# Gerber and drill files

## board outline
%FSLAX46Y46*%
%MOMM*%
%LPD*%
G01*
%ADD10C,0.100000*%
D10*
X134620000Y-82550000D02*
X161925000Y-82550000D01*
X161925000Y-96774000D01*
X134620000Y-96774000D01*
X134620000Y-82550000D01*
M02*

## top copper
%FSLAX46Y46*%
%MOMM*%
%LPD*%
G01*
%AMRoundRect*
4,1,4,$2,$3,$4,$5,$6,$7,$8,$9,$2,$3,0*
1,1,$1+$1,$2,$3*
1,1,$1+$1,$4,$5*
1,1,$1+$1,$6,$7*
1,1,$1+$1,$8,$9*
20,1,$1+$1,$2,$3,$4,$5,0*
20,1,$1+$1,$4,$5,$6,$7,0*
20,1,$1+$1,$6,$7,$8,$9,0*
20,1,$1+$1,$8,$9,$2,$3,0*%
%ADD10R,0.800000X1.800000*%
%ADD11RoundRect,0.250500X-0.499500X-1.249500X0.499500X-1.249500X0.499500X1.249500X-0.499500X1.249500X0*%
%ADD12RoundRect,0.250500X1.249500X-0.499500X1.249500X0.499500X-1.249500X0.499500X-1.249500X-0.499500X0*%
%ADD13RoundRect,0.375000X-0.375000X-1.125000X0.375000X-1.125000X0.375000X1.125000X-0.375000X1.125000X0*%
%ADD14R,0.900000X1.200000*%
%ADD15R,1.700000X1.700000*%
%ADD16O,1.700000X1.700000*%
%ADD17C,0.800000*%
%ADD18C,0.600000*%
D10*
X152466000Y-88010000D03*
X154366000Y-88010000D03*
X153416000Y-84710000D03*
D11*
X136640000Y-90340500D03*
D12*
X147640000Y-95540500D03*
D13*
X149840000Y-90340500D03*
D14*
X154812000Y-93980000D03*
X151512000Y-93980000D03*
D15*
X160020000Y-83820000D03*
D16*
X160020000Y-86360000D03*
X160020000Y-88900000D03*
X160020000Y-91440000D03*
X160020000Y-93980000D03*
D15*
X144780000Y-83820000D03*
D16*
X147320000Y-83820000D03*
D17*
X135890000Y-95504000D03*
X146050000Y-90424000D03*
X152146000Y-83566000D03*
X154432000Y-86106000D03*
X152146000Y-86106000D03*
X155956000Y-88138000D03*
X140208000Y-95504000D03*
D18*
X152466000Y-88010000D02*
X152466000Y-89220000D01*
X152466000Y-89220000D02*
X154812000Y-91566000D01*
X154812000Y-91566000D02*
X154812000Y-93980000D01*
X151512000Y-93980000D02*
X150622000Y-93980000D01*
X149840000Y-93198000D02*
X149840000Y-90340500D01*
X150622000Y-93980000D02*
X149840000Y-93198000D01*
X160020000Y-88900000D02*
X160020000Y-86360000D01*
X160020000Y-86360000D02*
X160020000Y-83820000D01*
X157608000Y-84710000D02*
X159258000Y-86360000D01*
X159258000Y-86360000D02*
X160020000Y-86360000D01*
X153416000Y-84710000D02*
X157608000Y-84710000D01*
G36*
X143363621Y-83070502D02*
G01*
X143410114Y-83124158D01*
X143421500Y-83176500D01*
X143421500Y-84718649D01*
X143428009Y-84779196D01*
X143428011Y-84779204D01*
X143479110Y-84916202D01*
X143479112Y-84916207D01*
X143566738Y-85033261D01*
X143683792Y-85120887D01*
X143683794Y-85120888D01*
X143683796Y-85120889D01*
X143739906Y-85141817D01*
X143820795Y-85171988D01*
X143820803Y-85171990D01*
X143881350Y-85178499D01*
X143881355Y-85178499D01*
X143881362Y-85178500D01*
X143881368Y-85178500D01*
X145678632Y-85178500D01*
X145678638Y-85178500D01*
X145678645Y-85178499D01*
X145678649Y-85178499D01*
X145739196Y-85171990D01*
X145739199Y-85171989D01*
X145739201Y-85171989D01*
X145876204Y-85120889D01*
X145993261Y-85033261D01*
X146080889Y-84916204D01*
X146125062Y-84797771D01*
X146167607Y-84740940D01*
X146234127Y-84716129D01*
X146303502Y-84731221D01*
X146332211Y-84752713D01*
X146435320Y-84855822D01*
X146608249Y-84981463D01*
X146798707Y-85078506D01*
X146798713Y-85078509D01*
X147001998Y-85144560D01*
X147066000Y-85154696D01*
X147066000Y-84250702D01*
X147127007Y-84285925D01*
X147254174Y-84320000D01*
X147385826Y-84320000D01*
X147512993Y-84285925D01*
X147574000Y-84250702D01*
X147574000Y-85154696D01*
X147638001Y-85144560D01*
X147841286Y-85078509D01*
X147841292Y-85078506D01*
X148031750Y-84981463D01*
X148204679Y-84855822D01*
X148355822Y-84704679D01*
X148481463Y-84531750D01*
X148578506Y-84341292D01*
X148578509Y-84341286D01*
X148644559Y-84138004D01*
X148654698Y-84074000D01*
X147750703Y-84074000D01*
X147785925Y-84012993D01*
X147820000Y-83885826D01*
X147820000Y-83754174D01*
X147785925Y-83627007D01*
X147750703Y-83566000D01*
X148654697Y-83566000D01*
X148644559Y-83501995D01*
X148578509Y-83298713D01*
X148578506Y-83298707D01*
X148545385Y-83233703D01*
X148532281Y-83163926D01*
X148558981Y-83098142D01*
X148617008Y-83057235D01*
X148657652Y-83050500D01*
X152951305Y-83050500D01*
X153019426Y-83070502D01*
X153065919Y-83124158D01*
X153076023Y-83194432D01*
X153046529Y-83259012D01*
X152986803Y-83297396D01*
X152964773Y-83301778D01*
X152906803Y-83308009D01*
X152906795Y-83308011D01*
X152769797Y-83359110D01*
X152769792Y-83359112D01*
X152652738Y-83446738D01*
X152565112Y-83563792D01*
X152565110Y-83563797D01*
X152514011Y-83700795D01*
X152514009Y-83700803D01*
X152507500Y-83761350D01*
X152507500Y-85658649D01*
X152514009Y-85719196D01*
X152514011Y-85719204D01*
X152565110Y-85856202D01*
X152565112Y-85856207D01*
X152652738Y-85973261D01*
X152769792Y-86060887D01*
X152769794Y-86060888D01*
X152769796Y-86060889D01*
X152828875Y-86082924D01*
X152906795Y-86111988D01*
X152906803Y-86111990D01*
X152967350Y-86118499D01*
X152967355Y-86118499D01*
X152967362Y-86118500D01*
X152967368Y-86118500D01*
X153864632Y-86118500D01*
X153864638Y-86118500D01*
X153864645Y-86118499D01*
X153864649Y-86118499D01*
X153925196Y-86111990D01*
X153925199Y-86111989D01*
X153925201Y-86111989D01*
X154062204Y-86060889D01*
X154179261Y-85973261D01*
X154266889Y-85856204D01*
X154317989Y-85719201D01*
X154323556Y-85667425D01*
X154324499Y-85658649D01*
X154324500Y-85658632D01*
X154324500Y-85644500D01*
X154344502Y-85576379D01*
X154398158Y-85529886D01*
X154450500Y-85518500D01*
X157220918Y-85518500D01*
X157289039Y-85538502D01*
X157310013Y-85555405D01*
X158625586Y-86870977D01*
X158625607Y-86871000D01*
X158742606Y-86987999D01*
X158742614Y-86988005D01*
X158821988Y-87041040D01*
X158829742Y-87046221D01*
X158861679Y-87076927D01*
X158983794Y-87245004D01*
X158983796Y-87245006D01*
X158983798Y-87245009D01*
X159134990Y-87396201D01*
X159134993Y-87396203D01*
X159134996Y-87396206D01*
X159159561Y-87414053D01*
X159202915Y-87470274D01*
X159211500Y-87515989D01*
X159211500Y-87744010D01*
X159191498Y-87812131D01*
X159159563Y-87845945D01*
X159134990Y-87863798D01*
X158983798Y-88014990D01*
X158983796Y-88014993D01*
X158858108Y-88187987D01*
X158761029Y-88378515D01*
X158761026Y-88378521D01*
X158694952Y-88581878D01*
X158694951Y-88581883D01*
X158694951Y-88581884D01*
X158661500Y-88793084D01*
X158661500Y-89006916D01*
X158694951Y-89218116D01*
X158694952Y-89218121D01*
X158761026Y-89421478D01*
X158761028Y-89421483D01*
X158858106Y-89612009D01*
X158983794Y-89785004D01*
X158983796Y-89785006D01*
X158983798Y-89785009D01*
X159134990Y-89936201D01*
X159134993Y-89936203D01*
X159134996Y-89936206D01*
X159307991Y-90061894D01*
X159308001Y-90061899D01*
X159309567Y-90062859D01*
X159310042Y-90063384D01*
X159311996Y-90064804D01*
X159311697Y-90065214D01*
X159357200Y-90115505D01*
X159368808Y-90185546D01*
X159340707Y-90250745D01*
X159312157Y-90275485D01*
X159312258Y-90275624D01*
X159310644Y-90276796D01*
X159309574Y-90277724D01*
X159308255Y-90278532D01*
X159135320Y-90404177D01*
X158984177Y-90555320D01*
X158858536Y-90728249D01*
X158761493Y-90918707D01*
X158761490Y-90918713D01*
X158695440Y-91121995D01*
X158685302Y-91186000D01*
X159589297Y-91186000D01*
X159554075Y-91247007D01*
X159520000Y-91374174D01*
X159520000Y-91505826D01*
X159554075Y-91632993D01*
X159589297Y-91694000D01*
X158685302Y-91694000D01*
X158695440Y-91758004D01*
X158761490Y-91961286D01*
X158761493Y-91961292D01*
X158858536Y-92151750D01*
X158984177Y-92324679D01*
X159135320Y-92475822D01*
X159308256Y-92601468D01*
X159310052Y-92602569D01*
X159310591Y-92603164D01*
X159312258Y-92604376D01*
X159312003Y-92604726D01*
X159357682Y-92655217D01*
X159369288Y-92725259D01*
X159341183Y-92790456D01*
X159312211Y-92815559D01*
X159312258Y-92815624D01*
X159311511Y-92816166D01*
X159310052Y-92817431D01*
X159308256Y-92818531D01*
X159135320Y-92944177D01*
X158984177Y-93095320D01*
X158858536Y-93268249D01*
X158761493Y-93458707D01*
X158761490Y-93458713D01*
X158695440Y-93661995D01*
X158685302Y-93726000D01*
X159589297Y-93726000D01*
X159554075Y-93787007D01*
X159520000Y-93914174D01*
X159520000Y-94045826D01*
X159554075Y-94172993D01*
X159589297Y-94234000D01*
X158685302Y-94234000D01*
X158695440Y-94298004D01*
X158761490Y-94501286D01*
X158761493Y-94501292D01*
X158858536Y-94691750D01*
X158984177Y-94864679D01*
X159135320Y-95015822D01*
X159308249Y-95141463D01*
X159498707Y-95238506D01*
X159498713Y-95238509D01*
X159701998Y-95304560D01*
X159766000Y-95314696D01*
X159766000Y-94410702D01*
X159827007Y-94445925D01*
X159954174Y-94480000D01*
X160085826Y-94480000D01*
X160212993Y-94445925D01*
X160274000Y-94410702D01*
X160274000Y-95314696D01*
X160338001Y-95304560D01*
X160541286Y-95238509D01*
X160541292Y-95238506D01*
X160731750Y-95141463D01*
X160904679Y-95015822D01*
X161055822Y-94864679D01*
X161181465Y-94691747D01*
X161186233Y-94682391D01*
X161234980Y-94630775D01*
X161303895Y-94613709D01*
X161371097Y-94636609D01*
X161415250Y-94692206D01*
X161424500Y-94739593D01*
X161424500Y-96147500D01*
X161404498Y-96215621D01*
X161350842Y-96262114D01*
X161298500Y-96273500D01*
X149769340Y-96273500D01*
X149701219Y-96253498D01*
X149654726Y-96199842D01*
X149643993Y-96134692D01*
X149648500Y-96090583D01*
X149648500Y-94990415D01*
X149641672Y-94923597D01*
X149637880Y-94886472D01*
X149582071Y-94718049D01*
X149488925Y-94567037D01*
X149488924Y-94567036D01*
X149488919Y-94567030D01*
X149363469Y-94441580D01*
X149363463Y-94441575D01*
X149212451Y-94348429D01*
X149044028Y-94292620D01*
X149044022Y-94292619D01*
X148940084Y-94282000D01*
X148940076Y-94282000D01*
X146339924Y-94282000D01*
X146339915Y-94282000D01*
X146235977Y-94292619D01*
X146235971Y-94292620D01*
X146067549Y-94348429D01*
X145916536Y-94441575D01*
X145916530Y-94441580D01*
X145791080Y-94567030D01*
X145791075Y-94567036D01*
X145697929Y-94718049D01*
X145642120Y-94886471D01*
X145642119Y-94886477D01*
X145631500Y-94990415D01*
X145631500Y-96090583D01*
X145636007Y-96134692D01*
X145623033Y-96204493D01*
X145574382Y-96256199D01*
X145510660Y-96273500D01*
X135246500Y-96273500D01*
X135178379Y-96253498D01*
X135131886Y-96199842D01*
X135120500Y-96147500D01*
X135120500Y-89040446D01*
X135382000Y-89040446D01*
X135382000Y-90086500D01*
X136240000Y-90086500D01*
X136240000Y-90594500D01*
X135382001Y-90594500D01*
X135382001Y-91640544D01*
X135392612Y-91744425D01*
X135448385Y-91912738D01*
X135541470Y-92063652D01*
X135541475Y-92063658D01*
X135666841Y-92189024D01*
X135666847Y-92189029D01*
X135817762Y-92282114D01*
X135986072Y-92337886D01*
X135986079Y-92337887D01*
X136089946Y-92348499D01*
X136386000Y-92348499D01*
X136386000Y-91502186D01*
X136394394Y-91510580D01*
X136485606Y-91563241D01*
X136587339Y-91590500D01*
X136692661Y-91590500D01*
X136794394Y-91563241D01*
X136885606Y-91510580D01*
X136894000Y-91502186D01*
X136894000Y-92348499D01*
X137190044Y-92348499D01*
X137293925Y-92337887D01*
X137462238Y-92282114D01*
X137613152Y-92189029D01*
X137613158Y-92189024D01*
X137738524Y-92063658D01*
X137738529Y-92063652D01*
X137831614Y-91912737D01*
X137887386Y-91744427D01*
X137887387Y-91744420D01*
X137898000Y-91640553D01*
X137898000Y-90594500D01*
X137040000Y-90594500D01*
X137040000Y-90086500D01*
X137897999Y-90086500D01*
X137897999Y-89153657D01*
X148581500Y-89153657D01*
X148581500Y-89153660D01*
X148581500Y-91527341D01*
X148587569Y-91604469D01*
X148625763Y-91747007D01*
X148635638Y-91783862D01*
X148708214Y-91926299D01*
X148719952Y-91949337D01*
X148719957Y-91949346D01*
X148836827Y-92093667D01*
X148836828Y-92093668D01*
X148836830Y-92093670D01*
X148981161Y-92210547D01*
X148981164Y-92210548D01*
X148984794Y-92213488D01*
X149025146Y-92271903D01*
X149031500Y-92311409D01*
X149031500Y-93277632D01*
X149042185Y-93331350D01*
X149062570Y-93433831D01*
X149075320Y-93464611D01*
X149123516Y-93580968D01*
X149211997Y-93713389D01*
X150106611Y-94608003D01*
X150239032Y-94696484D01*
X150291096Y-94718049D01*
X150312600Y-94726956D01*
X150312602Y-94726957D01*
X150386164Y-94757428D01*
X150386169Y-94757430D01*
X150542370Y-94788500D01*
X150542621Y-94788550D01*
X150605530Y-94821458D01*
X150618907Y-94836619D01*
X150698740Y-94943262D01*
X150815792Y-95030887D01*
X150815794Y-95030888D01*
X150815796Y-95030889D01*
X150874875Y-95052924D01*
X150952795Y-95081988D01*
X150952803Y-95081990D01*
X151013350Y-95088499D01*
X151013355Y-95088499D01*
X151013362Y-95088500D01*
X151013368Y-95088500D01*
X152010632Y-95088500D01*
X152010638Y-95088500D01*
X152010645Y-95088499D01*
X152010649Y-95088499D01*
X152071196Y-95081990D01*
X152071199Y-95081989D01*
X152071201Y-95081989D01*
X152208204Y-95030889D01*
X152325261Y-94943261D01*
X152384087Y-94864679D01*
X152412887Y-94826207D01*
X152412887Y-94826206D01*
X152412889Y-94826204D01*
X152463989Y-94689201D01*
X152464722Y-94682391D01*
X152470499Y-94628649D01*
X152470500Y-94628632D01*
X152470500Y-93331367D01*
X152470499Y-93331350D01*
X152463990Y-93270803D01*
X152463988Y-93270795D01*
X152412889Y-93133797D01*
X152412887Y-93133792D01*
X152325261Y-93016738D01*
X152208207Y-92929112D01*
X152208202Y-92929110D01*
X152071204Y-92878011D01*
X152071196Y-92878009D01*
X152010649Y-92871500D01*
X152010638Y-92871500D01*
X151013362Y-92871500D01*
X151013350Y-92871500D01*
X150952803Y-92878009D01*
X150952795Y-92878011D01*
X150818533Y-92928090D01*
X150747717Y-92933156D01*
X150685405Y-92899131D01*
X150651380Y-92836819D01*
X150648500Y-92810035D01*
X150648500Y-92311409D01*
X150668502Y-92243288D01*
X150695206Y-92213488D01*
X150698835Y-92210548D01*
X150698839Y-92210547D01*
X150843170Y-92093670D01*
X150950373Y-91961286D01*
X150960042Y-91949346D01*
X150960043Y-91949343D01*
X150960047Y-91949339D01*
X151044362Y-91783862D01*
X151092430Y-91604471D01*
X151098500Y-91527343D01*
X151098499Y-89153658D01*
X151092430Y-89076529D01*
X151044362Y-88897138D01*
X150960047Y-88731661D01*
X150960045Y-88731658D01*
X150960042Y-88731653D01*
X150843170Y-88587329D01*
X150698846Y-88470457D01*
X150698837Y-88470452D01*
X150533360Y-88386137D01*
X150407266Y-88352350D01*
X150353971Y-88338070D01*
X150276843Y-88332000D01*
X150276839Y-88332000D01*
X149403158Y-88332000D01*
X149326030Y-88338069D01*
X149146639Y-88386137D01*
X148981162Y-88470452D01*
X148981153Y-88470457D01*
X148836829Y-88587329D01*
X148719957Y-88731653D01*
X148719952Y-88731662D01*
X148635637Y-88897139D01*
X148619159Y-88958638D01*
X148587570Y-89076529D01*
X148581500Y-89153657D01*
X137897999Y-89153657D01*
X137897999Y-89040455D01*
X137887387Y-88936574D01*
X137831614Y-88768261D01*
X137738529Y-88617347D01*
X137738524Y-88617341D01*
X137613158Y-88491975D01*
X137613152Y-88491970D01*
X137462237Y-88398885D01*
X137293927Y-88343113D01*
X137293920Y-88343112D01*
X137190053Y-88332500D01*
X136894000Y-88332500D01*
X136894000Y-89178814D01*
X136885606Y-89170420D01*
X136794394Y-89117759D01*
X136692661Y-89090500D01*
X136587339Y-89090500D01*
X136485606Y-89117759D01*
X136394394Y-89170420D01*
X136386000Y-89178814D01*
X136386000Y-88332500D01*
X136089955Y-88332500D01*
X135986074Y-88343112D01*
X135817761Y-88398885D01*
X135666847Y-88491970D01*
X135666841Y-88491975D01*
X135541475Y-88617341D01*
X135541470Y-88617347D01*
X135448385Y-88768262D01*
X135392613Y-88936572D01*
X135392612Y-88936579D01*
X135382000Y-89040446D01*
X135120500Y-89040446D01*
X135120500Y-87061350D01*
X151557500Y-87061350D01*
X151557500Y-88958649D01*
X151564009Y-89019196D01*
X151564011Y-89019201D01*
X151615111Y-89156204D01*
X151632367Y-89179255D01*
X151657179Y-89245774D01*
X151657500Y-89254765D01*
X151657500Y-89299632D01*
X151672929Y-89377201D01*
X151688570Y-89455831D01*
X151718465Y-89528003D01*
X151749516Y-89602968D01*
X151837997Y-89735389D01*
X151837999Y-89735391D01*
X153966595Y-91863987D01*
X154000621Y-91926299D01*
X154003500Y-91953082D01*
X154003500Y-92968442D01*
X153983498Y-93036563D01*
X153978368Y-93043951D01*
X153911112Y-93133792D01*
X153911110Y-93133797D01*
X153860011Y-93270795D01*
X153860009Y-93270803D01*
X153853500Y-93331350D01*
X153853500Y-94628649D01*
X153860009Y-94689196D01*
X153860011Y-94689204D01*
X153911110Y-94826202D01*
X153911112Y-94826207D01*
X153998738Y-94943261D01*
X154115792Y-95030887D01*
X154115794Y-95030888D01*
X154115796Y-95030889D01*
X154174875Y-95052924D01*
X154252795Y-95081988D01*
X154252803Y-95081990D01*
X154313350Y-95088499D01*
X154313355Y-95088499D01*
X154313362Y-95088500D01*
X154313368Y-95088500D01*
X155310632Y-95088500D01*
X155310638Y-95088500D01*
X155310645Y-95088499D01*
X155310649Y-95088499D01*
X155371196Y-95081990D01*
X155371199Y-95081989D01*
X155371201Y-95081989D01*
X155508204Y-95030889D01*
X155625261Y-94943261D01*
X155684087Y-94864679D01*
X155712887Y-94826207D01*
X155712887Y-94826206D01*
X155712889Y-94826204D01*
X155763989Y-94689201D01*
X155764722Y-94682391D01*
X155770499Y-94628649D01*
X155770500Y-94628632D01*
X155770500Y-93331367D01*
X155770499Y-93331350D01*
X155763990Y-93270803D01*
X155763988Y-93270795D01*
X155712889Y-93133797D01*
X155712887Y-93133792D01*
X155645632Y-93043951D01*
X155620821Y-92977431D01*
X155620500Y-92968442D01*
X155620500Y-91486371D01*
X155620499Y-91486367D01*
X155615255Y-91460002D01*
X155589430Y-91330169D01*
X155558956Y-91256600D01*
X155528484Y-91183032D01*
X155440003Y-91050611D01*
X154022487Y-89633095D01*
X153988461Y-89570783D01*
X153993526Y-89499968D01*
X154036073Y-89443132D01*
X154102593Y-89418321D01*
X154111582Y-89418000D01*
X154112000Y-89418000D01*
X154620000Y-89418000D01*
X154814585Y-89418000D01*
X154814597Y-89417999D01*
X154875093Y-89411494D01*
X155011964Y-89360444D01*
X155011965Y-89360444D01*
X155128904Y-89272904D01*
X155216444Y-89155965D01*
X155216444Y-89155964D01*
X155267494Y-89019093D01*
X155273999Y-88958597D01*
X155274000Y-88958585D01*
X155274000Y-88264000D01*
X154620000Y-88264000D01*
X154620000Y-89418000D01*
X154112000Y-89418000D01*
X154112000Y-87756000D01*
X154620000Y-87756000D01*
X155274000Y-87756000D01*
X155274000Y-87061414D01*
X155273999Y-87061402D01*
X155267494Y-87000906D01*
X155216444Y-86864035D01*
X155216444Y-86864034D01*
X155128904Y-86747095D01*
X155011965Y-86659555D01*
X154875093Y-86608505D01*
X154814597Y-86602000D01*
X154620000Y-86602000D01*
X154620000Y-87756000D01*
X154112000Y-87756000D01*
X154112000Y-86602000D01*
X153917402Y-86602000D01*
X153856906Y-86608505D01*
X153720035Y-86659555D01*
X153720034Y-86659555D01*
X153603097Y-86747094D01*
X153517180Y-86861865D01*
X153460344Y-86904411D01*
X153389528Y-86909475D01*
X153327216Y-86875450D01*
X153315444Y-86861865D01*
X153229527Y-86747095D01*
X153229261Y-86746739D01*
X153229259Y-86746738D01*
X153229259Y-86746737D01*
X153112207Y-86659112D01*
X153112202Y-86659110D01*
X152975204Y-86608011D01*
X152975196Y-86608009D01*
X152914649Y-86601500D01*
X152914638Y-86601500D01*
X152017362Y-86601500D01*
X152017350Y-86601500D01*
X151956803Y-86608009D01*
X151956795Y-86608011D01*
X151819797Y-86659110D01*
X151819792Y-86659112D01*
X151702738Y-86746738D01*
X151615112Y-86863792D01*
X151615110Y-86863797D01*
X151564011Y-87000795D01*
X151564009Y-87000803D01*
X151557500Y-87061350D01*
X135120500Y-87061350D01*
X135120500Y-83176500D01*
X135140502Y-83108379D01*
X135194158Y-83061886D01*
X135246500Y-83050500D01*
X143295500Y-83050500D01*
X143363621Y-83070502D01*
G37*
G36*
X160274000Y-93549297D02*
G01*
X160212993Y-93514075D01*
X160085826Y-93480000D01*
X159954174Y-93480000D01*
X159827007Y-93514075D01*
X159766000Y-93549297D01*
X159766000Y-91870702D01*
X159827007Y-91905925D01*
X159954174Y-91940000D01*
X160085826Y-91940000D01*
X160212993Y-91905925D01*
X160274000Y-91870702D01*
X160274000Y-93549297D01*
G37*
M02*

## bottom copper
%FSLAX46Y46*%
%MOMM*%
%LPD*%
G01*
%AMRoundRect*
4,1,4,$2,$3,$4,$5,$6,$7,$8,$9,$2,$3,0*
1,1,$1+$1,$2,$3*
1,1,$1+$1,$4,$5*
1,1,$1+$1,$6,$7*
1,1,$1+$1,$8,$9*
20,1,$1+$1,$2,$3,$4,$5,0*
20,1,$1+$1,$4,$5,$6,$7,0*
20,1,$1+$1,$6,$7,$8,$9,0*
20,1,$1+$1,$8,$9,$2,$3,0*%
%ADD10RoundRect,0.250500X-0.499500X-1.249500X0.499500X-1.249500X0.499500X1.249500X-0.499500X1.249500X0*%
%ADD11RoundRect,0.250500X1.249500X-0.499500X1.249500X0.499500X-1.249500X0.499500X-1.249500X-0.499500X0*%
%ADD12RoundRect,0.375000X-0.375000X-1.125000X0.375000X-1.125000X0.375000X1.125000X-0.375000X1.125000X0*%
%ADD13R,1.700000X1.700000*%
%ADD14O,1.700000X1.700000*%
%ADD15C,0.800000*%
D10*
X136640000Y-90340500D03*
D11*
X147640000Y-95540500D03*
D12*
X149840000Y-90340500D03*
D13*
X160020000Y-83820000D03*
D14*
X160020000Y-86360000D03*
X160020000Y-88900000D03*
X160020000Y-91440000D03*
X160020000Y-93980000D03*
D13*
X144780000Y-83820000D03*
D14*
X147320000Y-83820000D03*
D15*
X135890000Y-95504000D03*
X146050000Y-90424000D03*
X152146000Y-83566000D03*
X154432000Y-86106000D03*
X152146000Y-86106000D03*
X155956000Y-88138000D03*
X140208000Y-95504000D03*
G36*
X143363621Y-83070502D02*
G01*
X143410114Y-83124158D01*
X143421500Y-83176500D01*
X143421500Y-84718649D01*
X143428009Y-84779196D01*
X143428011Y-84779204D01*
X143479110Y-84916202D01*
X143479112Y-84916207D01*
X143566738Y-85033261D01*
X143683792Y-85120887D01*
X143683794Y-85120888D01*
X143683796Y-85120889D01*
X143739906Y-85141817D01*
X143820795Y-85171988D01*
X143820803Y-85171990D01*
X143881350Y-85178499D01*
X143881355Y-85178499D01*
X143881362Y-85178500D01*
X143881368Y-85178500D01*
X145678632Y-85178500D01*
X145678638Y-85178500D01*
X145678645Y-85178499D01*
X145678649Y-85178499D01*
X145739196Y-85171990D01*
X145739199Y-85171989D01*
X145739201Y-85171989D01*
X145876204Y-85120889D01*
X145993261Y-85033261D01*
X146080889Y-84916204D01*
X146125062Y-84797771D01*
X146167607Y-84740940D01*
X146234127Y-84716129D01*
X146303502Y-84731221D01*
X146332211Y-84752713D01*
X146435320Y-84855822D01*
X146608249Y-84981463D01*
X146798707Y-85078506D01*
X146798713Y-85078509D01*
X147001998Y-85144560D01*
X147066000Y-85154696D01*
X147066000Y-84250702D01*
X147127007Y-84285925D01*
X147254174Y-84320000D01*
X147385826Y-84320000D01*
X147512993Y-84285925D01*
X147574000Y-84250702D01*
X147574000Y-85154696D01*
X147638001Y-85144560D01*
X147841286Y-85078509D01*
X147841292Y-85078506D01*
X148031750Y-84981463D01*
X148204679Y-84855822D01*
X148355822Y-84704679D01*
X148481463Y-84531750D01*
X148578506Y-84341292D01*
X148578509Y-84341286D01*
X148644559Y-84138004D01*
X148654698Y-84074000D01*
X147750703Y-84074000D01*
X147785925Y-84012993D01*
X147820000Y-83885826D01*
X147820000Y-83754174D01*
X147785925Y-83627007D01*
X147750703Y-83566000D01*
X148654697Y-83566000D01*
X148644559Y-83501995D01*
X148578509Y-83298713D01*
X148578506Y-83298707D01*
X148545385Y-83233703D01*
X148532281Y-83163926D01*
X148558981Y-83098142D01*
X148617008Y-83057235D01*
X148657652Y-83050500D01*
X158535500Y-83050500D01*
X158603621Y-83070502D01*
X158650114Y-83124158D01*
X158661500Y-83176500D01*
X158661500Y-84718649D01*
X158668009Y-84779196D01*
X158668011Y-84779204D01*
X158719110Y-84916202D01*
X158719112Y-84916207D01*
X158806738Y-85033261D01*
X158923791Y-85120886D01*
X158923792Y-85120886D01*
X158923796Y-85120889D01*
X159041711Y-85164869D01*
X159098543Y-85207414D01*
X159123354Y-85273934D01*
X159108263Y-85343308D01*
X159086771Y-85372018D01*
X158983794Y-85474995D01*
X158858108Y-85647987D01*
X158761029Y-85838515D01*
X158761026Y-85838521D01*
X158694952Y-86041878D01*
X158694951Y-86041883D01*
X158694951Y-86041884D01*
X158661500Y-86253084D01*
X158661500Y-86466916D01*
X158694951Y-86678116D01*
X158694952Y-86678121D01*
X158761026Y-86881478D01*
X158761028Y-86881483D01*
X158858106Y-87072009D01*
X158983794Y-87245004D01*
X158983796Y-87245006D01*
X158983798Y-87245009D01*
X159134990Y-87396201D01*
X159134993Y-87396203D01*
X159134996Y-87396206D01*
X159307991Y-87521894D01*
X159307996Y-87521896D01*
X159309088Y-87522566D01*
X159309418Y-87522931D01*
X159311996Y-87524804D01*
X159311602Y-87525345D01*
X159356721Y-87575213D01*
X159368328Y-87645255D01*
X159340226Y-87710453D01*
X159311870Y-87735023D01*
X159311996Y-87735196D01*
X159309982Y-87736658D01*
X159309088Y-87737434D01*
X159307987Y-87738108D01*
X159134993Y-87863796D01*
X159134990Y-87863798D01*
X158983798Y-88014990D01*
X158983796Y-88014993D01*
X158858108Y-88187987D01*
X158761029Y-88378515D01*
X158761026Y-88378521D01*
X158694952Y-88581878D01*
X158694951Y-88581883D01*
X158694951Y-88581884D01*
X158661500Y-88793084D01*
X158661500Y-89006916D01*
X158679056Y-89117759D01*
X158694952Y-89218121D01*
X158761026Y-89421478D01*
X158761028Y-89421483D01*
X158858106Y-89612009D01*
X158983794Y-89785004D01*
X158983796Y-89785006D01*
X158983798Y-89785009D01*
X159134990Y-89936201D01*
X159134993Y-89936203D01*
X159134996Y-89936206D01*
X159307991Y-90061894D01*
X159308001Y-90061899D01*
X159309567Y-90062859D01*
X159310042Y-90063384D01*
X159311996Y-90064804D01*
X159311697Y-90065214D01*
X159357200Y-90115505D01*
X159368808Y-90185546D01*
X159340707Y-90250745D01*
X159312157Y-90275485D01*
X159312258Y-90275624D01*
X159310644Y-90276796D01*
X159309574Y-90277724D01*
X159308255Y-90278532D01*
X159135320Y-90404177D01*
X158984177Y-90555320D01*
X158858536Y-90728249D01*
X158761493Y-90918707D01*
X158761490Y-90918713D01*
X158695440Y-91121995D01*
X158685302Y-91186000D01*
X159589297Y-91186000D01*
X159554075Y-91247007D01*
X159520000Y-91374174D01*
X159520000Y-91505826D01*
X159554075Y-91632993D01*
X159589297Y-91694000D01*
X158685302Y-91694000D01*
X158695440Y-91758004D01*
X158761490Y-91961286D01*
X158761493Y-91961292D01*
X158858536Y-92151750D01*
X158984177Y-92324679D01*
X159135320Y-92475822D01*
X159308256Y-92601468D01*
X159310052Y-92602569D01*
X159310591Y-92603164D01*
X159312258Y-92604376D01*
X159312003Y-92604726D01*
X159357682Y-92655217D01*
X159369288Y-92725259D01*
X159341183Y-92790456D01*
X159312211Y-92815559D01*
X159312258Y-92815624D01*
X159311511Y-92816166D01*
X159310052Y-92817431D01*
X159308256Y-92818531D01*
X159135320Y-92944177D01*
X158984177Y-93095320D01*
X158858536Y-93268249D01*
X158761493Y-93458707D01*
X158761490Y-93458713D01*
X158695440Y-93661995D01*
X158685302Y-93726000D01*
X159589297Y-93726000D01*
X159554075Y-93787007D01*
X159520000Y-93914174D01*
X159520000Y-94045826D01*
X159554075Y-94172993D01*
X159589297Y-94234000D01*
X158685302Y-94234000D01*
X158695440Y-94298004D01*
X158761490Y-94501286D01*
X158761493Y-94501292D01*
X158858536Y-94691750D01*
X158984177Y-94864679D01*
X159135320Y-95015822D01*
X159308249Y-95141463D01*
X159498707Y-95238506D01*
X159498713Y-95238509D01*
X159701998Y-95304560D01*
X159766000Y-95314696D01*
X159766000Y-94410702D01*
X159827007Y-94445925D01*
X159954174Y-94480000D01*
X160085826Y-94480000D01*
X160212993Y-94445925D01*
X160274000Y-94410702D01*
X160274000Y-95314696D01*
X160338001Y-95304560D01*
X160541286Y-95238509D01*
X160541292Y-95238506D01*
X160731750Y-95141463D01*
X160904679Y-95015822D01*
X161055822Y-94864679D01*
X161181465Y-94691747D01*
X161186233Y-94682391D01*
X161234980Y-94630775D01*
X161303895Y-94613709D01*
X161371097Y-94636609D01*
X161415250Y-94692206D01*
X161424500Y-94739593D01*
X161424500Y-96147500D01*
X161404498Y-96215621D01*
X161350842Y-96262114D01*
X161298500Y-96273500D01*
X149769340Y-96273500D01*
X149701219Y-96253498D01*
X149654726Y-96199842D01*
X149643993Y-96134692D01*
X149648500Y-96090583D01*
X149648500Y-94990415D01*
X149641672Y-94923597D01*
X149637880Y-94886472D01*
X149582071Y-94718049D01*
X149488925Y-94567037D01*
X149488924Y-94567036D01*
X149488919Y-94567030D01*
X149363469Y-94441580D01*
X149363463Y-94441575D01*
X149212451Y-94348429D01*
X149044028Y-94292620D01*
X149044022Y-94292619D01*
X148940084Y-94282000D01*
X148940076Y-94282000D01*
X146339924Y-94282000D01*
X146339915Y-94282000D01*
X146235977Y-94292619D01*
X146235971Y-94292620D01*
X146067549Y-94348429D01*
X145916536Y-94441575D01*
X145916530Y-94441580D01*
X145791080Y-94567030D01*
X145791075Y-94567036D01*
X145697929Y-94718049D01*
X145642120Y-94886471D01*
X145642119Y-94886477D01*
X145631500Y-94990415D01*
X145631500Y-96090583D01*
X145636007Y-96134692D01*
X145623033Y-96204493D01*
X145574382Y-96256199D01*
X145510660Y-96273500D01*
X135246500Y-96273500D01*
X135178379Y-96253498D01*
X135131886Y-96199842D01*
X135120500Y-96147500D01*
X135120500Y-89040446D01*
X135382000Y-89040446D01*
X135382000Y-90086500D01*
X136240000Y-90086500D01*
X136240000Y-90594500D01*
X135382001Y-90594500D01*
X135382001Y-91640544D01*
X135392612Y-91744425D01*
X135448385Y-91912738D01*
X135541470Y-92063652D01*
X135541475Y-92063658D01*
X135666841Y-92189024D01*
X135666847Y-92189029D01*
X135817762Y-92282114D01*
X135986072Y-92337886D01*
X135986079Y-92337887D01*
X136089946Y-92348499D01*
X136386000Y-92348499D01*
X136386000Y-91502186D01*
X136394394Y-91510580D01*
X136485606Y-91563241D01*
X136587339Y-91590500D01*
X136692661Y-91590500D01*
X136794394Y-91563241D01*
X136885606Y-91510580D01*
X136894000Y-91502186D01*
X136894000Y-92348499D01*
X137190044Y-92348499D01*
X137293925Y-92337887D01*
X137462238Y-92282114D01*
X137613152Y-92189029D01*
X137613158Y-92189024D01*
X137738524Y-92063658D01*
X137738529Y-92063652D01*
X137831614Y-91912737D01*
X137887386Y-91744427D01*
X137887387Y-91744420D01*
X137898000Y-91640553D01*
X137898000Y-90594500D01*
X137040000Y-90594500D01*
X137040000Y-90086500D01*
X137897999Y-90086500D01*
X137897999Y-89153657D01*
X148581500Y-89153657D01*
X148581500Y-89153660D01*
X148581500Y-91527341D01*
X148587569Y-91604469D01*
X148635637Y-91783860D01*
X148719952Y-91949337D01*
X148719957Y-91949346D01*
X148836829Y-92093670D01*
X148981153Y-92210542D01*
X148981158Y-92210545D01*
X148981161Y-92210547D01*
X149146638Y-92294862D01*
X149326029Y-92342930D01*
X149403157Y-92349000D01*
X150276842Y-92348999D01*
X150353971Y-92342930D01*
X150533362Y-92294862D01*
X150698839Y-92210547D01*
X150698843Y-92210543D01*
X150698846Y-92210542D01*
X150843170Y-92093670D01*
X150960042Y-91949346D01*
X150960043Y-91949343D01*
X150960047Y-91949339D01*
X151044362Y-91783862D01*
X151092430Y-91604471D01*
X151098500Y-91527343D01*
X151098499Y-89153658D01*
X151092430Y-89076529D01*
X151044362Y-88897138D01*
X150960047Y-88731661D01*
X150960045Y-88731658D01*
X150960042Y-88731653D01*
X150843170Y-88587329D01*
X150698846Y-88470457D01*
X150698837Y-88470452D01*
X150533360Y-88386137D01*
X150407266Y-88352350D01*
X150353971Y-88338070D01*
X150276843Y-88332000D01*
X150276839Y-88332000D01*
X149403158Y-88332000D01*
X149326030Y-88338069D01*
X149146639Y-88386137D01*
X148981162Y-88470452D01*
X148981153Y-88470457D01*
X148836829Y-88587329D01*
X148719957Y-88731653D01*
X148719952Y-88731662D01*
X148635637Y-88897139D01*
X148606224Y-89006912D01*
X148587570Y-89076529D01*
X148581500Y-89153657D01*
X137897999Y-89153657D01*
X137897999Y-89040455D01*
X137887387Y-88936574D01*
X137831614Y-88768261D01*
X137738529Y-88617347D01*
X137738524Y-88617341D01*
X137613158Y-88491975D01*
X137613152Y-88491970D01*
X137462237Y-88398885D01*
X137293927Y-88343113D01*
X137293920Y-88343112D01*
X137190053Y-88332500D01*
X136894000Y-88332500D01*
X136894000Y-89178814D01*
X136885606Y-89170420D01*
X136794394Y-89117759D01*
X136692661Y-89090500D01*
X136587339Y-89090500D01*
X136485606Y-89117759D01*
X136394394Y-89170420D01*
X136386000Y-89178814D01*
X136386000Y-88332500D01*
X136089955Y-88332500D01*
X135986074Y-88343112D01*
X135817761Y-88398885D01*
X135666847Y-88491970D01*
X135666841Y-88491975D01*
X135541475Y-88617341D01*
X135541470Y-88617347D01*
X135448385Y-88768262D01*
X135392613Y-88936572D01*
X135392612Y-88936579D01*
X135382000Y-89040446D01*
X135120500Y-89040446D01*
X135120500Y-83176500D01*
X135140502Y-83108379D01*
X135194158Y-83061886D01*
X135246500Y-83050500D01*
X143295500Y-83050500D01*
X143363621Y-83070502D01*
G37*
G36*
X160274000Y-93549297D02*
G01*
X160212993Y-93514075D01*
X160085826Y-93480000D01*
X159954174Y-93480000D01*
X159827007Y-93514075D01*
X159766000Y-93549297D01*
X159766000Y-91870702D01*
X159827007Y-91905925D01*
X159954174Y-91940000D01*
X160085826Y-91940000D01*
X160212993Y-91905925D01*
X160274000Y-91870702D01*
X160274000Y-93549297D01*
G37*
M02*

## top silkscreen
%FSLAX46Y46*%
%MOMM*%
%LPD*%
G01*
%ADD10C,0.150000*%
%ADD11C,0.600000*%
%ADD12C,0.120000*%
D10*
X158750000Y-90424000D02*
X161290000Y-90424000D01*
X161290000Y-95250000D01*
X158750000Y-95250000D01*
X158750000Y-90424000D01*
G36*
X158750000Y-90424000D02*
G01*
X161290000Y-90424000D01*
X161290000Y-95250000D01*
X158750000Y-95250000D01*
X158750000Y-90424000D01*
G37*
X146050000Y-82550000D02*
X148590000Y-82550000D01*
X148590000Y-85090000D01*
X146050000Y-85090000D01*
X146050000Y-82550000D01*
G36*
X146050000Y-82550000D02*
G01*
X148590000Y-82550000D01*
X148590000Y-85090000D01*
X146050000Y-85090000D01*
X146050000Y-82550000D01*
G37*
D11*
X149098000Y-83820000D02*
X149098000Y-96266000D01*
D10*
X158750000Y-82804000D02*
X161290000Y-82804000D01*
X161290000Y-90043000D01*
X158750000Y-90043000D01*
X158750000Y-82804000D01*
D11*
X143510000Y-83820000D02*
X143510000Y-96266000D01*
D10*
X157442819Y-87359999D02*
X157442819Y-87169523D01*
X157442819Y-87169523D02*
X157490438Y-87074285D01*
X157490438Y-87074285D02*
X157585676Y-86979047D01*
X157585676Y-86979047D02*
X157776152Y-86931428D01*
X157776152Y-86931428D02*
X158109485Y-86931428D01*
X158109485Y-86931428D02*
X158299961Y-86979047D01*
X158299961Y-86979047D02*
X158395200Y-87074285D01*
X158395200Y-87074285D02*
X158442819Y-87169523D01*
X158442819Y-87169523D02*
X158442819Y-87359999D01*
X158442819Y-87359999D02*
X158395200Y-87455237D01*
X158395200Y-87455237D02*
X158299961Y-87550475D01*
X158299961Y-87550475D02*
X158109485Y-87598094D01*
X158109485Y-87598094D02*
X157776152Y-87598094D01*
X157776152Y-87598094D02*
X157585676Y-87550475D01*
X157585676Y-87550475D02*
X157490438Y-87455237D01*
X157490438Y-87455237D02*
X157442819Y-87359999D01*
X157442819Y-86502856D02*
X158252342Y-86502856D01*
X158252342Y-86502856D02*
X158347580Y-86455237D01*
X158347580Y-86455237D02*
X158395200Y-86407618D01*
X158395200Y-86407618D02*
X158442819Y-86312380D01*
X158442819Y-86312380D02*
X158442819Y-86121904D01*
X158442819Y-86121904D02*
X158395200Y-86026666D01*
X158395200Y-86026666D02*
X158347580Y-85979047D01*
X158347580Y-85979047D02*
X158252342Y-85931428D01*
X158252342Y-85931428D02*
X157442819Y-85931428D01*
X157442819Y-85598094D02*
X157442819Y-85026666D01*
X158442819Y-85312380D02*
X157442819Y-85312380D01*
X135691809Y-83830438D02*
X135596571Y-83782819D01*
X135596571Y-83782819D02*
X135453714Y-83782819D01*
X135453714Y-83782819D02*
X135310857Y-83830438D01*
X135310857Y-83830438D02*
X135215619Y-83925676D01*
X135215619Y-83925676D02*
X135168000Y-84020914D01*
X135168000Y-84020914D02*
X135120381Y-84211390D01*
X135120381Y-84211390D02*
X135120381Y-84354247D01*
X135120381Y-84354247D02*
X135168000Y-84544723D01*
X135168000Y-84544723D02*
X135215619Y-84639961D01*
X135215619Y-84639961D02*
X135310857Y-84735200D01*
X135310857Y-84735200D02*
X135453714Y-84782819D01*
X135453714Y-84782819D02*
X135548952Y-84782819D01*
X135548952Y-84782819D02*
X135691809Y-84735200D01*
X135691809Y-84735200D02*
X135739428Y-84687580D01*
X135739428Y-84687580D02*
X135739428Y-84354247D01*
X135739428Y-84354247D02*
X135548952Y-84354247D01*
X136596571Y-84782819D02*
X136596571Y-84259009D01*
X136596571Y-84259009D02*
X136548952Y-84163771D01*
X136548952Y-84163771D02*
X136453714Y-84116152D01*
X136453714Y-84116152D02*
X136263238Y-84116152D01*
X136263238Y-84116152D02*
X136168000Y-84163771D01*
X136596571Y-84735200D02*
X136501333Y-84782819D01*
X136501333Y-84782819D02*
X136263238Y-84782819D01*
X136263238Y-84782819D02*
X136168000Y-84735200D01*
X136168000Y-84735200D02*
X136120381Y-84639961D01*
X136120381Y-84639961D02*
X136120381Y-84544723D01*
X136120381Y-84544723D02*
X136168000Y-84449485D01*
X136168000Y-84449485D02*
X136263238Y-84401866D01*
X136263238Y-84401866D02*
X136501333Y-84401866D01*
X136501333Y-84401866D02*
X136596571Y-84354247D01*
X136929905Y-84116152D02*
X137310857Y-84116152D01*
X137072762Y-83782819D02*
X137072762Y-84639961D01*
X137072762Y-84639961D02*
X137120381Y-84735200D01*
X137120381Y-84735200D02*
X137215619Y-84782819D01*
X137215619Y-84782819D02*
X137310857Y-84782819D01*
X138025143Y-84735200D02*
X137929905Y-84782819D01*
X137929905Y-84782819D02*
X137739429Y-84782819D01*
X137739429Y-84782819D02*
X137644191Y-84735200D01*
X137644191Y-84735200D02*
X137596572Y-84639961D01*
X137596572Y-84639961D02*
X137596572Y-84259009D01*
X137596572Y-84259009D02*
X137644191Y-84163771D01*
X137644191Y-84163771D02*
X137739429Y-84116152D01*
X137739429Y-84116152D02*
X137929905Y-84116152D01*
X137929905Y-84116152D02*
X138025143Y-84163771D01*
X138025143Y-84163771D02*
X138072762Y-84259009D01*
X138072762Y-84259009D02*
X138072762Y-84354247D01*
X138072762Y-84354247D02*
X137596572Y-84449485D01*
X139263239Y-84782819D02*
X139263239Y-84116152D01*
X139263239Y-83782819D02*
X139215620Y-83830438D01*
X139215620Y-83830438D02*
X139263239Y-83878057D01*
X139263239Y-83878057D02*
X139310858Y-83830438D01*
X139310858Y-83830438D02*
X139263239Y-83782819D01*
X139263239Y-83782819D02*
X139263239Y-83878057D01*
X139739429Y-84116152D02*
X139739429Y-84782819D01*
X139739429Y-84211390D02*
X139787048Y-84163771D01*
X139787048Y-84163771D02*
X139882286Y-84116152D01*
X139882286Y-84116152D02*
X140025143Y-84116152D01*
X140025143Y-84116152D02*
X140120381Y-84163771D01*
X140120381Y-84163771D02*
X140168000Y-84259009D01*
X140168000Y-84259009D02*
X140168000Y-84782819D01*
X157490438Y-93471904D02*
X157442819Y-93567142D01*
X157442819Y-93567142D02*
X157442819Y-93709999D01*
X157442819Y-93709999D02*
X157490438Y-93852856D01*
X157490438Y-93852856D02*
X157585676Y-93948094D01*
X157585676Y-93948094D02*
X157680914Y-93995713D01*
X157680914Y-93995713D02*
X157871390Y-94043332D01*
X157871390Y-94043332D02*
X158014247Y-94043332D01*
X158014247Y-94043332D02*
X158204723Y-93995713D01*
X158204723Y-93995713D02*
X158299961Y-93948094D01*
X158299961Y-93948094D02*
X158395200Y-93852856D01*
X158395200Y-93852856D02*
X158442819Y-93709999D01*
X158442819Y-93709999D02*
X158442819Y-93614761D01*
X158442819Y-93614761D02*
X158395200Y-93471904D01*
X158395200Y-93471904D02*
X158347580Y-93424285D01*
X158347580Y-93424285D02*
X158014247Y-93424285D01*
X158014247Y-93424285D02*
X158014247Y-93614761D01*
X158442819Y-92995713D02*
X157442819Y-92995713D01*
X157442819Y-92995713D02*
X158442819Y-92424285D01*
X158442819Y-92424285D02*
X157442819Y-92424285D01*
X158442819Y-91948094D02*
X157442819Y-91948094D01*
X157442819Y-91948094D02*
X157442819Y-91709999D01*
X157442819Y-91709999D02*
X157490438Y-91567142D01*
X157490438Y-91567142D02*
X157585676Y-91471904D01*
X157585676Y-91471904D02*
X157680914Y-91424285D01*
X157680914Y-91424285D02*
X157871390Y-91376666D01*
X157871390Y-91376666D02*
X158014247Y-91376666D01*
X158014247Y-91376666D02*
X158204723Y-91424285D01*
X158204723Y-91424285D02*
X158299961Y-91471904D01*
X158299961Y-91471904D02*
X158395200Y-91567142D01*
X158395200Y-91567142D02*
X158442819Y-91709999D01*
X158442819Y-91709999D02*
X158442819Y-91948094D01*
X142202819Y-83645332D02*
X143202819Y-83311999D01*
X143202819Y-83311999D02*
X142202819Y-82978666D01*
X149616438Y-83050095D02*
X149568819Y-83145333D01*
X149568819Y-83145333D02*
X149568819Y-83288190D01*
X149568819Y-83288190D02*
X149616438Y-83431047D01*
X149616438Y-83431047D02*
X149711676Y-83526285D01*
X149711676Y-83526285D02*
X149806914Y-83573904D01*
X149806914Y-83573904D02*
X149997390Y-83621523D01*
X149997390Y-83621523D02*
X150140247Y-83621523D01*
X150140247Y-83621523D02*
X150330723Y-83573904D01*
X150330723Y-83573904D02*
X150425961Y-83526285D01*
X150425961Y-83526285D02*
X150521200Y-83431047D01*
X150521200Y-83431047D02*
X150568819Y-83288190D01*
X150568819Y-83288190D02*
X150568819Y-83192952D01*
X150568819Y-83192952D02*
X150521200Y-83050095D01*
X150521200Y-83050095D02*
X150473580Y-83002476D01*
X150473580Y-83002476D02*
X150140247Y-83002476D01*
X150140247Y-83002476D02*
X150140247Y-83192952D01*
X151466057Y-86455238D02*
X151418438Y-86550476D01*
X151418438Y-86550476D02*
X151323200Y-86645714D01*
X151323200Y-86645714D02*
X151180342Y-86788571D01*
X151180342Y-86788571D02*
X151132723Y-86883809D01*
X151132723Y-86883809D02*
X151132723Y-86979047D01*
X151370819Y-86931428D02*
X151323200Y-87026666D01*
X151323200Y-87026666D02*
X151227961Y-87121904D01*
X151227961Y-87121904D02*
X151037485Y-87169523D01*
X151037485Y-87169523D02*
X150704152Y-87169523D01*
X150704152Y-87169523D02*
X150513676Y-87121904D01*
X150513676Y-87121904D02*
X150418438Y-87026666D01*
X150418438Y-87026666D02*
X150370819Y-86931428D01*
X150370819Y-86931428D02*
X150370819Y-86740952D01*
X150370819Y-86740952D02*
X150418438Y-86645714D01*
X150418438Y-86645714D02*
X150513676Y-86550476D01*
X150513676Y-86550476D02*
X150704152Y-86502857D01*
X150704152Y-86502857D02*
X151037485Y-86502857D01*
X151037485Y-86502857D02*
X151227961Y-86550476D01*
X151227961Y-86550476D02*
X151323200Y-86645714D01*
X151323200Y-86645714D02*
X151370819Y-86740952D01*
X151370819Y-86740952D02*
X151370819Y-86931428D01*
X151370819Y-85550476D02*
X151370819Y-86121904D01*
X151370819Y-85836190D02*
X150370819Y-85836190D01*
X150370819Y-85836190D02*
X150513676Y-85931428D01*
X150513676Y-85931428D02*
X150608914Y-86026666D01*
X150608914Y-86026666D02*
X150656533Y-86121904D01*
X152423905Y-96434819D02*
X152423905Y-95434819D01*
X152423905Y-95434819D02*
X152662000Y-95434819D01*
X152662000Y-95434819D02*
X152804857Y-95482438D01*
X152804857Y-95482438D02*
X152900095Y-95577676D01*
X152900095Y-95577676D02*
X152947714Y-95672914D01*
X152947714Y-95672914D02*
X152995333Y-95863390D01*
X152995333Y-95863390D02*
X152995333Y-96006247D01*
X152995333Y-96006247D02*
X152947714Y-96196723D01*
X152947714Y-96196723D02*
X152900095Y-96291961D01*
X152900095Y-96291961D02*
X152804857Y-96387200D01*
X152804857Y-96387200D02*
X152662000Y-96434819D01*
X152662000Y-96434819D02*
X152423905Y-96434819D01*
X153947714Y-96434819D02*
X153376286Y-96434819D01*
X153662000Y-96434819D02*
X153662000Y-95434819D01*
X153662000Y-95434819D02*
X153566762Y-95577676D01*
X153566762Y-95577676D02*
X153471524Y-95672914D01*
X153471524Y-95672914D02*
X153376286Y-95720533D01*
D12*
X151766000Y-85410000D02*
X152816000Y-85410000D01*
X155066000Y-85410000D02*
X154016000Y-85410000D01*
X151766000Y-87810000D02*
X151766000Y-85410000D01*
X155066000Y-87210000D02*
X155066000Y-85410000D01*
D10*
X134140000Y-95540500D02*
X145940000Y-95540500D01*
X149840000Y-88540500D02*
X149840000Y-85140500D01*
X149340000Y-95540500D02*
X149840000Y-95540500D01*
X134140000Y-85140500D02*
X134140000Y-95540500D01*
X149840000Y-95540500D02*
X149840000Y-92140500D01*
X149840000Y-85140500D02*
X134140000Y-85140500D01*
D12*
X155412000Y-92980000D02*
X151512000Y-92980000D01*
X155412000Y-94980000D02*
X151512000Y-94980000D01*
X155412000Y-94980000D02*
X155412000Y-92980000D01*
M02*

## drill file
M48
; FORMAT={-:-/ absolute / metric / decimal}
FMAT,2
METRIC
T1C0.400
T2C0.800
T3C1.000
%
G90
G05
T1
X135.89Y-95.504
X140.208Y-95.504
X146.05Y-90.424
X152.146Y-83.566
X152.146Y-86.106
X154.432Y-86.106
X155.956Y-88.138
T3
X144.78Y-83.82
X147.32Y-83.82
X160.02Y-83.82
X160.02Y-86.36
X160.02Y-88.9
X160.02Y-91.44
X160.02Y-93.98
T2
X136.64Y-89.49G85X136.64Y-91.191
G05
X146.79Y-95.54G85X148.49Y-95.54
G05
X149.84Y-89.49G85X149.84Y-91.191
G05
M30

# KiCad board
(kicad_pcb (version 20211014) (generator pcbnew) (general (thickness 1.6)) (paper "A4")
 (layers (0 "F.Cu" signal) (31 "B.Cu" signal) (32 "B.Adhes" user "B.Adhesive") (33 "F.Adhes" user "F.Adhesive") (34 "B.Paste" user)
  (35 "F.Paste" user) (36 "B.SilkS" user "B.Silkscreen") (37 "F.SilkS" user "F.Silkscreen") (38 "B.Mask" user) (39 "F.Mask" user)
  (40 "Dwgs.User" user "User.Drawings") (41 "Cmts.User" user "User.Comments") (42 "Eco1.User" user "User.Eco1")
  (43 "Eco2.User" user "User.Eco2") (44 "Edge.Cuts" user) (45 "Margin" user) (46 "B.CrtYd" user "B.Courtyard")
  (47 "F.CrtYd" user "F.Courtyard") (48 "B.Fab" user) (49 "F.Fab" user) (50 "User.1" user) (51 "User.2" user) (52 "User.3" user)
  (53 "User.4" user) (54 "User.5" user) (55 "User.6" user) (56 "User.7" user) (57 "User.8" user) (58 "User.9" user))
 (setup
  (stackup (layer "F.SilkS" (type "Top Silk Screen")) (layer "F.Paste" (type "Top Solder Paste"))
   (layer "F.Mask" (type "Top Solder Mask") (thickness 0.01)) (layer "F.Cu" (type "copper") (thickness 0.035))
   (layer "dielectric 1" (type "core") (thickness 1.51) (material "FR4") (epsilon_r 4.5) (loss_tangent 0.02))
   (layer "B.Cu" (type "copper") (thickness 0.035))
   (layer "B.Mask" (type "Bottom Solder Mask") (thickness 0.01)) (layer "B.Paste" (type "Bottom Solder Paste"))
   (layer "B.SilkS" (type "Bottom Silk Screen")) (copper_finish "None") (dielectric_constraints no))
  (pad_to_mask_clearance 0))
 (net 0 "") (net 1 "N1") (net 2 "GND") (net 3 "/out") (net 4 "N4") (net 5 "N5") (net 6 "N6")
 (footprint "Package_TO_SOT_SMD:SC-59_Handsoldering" (layer "F.Cu") (at 153.416 86.36 90)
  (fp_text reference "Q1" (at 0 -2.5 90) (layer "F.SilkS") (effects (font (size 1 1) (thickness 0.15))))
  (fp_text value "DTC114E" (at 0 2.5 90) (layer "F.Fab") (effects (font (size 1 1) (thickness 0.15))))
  (fp_line (start 0.95 -1.65) (end 0.95 -0.6) (layer "F.SilkS") (width 0.12))
  (fp_line (start 0.95 1.65) (end 0.95 0.6) (layer "F.SilkS") (width 0.12))
  (fp_line (start -1.45 -1.65) (end 0.95 -1.65) (layer "F.SilkS") (width 0.12))
  (fp_line (start -0.85 1.65) (end 0.95 1.65) (layer "F.SilkS") (width 0.12))
  (pad "1" smd rect (at -1.65 -0.95 90) (size 1.8 0.8) (layers "F.Cu" "F.Paste" "F.Mask") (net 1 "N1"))
  (pad "2" smd rect (at -1.65 0.95 90) (size 1.8 0.8) (layers "F.Cu" "F.Paste" "F.Mask") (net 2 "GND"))
  (pad "3" smd rect (at 1.65 0 90) (size 1.8 0.8) (layers "F.Cu" "F.Paste" "F.Mask") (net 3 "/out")))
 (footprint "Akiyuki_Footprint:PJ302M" (layer "F.Cu") (at 134.14 90.3405)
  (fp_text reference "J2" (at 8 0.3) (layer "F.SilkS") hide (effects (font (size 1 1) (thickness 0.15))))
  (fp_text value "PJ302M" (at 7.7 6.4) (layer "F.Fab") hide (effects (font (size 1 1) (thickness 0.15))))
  (fp_line (start 0 5.2) (end 11.8 5.2) (layer "F.SilkS") (width 0.15))
  (fp_line (start 15.7 -1.8) (end 15.7 -5.2) (layer "F.SilkS") (width 0.15))
  (fp_line (start 15.2 5.2) (end 15.7 5.2) (layer "F.SilkS") (width 0.15))
  (fp_line (start 0 -5.2) (end 0 5.2) (layer "F.SilkS") (width 0.15))
  (fp_line (start 15.7 5.2) (end 15.7 1.8) (layer "F.SilkS") (width 0.15))
  (fp_line (start 15.7 -5.2) (end 0 -5.2) (layer "F.SilkS") (width 0.15))
  (pad "1" thru_hole roundrect locked (at 2.5 0) (size 1.5 3) (drill oval 0.8 2.5) (layers *.Cu *.Mask) (roundrect_rratio 0.167)
   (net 2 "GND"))
  (pad "2" thru_hole roundrect locked (at 13.5 5.2 90) (size 1.5 3) (drill oval 0.8 2.5) (layers *.Cu *.Mask) (roundrect_rratio 0.167)
   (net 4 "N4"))
  (pad "3" thru_hole roundrect locked (at 15.7 0) (size 1.5 3) (drill oval 0.8 2.5) (layers *.Cu *.Mask) (roundrect_rratio 0.25)
   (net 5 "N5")))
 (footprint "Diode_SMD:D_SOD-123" (layer "F.Cu") (at 153.162 93.98 180)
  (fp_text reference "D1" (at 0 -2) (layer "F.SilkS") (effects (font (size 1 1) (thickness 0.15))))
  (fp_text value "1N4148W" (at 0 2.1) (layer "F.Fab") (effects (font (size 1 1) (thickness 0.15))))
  (fp_line (start -2.25 1) (end 1.65 1) (layer "F.SilkS") (width 0.12))
  (fp_line (start -2.25 -1) (end 1.65 -1) (layer "F.SilkS") (width 0.12))
  (fp_line (start -2.25 -1) (end -2.25 1) (layer "F.SilkS") (width 0.12))
  (pad "1" smd rect (at -1.65 0 180) (size 0.9 1.2) (layers "F.Cu" "F.Paste" "F.Mask") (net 1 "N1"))
  (pad "2" smd rect (at 1.65 0 180) (size 0.9 1.2) (layers "F.Cu" "F.Paste" "F.Mask") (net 5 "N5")))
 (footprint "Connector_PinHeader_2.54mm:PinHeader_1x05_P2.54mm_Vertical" (layer "B.Cu") (at 160.02 83.82 180)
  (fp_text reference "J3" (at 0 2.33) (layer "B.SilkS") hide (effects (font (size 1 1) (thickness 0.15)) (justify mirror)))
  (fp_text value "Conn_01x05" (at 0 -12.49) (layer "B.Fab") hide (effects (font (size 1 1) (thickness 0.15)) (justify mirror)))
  (pad "1" thru_hole rect (at 0 0 180) (size 1.7 1.7) (drill 1) (layers *.Cu *.Mask) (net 3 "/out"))
  (pad "2" thru_hole oval (at 0 -2.54 180) (size 1.7 1.7) (drill 1) (layers *.Cu *.Mask) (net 3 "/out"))
  (pad "3" thru_hole oval (at 0 -5.08 180) (size 1.7 1.7) (drill 1) (layers *.Cu *.Mask) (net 3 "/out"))
  (pad "4" thru_hole oval (at 0 -7.62 180) (size 1.7 1.7) (drill 1) (layers *.Cu *.Mask) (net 2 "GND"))
  (pad "5" thru_hole oval (at 0 -10.16 180) (size 1.7 1.7) (drill 1) (layers *.Cu *.Mask) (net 2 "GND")))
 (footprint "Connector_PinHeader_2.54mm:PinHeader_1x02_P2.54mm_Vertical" (layer "B.Cu") (at 144.78 83.82 -90)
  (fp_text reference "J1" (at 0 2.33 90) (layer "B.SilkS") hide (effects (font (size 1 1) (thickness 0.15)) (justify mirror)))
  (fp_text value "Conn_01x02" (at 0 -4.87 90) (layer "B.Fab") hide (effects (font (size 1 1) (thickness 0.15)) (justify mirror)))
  (pad "1" thru_hole rect (at 0 0 270) (size 1.7 1.7) (drill 1) (layers *.Cu *.Mask) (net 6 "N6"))
  (pad "2" thru_hole oval (at 0 -2.54 270) (size 1.7 1.7) (drill 1) (layers *.Cu *.Mask) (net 2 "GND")))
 (gr_rect (start 158.75 90.424) (end 161.29 95.25) (layer "F.SilkS") (width 0.15) (fill solid))
 (gr_rect (start 146.05 82.55) (end 148.59 85.09) (layer "F.SilkS") (width 0.15) (fill solid))
 (gr_line (start 149.098 83.82) (end 149.098 96.266) (layer "F.SilkS") (width 0.6))
 (gr_rect (start 158.75 82.804) (end 161.29 90.043) (layer "F.SilkS") (width 0.15) (fill none))
 (gr_line (start 143.51 83.82) (end 143.51 96.266) (layer "F.SilkS") (width 0.6))
 (gr_rect (start 161.925 82.55) (end 134.62 96.774) (layer "Edge.Cuts") (width 0.1) (fill none))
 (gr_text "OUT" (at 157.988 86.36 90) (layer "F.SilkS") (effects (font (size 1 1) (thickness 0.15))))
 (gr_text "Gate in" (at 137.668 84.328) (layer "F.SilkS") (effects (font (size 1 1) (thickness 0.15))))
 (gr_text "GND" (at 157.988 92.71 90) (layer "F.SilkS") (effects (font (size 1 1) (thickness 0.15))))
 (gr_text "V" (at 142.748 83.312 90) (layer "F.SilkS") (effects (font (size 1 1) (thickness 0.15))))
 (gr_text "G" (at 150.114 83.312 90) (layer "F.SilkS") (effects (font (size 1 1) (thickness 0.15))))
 (segment (start 152.466 88.01) (end 152.466 89.22) (width 0.6) (layer "F.Cu") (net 1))
 (segment (start 152.466 89.22) (end 154.812 91.566) (width 0.6) (layer "F.Cu") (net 1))
 (segment (start 154.812 91.566) (end 154.812 93.98) (width 0.6) (layer "F.Cu") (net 1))
 (segment (start 151.512 93.98) (end 150.622 93.98) (width 0.6) (layer "F.Cu") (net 5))
 (segment (start 149.84 93.198) (end 149.84 90.3405) (width 0.6) (layer "F.Cu") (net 5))
 (segment (start 150.622 93.98) (end 149.84 93.198) (width 0.6) (layer "F.Cu") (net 5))
 (via (at 135.89 95.504) (size 0.8) (drill 0.4) (layers "F.Cu" "B.Cu") (free) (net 2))
 (via (at 146.05 90.424) (size 0.8) (drill 0.4) (layers "F.Cu" "B.Cu") (free) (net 2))
 (via (at 152.146 83.566) (size 0.8) (drill 0.4) (layers "F.Cu" "B.Cu") (free) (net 2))
 (via (at 154.432 86.106) (size 0.8) (drill 0.4) (layers "F.Cu" "B.Cu") (free) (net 2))
 (via (at 152.146 86.106) (size 0.8) (drill 0.4) (layers "F.Cu" "B.Cu") (free) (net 2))
 (via (at 155.956 88.138) (size 0.8) (drill 0.4) (layers "F.Cu" "B.Cu") (free) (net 2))
 (via (at 140.208 95.504) (size 0.8) (drill 0.4) (layers "F.Cu" "B.Cu") (free) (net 2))
 (segment (start 160.02 88.9) (end 160.02 86.36) (width 0.6) (layer "F.Cu") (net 3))
 (segment (start 160.02 86.36) (end 160.02 83.82) (width 0.6) (layer "F.Cu") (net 3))
 (segment (start 157.608 84.71) (end 159.258 86.36) (width 0.6) (layer "F.Cu") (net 3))
 (segment (start 159.258 86.36) (end 160.02 86.36) (width 0.6) (layer "F.Cu") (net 3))
 (segment (start 153.416 84.71) (end 157.608 84.71) (width 0.6) (layer "F.Cu") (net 3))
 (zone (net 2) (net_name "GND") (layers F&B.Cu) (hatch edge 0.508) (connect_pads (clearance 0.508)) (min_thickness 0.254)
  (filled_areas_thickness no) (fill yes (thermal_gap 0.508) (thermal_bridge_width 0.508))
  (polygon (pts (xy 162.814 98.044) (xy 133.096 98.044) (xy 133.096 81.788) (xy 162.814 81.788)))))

